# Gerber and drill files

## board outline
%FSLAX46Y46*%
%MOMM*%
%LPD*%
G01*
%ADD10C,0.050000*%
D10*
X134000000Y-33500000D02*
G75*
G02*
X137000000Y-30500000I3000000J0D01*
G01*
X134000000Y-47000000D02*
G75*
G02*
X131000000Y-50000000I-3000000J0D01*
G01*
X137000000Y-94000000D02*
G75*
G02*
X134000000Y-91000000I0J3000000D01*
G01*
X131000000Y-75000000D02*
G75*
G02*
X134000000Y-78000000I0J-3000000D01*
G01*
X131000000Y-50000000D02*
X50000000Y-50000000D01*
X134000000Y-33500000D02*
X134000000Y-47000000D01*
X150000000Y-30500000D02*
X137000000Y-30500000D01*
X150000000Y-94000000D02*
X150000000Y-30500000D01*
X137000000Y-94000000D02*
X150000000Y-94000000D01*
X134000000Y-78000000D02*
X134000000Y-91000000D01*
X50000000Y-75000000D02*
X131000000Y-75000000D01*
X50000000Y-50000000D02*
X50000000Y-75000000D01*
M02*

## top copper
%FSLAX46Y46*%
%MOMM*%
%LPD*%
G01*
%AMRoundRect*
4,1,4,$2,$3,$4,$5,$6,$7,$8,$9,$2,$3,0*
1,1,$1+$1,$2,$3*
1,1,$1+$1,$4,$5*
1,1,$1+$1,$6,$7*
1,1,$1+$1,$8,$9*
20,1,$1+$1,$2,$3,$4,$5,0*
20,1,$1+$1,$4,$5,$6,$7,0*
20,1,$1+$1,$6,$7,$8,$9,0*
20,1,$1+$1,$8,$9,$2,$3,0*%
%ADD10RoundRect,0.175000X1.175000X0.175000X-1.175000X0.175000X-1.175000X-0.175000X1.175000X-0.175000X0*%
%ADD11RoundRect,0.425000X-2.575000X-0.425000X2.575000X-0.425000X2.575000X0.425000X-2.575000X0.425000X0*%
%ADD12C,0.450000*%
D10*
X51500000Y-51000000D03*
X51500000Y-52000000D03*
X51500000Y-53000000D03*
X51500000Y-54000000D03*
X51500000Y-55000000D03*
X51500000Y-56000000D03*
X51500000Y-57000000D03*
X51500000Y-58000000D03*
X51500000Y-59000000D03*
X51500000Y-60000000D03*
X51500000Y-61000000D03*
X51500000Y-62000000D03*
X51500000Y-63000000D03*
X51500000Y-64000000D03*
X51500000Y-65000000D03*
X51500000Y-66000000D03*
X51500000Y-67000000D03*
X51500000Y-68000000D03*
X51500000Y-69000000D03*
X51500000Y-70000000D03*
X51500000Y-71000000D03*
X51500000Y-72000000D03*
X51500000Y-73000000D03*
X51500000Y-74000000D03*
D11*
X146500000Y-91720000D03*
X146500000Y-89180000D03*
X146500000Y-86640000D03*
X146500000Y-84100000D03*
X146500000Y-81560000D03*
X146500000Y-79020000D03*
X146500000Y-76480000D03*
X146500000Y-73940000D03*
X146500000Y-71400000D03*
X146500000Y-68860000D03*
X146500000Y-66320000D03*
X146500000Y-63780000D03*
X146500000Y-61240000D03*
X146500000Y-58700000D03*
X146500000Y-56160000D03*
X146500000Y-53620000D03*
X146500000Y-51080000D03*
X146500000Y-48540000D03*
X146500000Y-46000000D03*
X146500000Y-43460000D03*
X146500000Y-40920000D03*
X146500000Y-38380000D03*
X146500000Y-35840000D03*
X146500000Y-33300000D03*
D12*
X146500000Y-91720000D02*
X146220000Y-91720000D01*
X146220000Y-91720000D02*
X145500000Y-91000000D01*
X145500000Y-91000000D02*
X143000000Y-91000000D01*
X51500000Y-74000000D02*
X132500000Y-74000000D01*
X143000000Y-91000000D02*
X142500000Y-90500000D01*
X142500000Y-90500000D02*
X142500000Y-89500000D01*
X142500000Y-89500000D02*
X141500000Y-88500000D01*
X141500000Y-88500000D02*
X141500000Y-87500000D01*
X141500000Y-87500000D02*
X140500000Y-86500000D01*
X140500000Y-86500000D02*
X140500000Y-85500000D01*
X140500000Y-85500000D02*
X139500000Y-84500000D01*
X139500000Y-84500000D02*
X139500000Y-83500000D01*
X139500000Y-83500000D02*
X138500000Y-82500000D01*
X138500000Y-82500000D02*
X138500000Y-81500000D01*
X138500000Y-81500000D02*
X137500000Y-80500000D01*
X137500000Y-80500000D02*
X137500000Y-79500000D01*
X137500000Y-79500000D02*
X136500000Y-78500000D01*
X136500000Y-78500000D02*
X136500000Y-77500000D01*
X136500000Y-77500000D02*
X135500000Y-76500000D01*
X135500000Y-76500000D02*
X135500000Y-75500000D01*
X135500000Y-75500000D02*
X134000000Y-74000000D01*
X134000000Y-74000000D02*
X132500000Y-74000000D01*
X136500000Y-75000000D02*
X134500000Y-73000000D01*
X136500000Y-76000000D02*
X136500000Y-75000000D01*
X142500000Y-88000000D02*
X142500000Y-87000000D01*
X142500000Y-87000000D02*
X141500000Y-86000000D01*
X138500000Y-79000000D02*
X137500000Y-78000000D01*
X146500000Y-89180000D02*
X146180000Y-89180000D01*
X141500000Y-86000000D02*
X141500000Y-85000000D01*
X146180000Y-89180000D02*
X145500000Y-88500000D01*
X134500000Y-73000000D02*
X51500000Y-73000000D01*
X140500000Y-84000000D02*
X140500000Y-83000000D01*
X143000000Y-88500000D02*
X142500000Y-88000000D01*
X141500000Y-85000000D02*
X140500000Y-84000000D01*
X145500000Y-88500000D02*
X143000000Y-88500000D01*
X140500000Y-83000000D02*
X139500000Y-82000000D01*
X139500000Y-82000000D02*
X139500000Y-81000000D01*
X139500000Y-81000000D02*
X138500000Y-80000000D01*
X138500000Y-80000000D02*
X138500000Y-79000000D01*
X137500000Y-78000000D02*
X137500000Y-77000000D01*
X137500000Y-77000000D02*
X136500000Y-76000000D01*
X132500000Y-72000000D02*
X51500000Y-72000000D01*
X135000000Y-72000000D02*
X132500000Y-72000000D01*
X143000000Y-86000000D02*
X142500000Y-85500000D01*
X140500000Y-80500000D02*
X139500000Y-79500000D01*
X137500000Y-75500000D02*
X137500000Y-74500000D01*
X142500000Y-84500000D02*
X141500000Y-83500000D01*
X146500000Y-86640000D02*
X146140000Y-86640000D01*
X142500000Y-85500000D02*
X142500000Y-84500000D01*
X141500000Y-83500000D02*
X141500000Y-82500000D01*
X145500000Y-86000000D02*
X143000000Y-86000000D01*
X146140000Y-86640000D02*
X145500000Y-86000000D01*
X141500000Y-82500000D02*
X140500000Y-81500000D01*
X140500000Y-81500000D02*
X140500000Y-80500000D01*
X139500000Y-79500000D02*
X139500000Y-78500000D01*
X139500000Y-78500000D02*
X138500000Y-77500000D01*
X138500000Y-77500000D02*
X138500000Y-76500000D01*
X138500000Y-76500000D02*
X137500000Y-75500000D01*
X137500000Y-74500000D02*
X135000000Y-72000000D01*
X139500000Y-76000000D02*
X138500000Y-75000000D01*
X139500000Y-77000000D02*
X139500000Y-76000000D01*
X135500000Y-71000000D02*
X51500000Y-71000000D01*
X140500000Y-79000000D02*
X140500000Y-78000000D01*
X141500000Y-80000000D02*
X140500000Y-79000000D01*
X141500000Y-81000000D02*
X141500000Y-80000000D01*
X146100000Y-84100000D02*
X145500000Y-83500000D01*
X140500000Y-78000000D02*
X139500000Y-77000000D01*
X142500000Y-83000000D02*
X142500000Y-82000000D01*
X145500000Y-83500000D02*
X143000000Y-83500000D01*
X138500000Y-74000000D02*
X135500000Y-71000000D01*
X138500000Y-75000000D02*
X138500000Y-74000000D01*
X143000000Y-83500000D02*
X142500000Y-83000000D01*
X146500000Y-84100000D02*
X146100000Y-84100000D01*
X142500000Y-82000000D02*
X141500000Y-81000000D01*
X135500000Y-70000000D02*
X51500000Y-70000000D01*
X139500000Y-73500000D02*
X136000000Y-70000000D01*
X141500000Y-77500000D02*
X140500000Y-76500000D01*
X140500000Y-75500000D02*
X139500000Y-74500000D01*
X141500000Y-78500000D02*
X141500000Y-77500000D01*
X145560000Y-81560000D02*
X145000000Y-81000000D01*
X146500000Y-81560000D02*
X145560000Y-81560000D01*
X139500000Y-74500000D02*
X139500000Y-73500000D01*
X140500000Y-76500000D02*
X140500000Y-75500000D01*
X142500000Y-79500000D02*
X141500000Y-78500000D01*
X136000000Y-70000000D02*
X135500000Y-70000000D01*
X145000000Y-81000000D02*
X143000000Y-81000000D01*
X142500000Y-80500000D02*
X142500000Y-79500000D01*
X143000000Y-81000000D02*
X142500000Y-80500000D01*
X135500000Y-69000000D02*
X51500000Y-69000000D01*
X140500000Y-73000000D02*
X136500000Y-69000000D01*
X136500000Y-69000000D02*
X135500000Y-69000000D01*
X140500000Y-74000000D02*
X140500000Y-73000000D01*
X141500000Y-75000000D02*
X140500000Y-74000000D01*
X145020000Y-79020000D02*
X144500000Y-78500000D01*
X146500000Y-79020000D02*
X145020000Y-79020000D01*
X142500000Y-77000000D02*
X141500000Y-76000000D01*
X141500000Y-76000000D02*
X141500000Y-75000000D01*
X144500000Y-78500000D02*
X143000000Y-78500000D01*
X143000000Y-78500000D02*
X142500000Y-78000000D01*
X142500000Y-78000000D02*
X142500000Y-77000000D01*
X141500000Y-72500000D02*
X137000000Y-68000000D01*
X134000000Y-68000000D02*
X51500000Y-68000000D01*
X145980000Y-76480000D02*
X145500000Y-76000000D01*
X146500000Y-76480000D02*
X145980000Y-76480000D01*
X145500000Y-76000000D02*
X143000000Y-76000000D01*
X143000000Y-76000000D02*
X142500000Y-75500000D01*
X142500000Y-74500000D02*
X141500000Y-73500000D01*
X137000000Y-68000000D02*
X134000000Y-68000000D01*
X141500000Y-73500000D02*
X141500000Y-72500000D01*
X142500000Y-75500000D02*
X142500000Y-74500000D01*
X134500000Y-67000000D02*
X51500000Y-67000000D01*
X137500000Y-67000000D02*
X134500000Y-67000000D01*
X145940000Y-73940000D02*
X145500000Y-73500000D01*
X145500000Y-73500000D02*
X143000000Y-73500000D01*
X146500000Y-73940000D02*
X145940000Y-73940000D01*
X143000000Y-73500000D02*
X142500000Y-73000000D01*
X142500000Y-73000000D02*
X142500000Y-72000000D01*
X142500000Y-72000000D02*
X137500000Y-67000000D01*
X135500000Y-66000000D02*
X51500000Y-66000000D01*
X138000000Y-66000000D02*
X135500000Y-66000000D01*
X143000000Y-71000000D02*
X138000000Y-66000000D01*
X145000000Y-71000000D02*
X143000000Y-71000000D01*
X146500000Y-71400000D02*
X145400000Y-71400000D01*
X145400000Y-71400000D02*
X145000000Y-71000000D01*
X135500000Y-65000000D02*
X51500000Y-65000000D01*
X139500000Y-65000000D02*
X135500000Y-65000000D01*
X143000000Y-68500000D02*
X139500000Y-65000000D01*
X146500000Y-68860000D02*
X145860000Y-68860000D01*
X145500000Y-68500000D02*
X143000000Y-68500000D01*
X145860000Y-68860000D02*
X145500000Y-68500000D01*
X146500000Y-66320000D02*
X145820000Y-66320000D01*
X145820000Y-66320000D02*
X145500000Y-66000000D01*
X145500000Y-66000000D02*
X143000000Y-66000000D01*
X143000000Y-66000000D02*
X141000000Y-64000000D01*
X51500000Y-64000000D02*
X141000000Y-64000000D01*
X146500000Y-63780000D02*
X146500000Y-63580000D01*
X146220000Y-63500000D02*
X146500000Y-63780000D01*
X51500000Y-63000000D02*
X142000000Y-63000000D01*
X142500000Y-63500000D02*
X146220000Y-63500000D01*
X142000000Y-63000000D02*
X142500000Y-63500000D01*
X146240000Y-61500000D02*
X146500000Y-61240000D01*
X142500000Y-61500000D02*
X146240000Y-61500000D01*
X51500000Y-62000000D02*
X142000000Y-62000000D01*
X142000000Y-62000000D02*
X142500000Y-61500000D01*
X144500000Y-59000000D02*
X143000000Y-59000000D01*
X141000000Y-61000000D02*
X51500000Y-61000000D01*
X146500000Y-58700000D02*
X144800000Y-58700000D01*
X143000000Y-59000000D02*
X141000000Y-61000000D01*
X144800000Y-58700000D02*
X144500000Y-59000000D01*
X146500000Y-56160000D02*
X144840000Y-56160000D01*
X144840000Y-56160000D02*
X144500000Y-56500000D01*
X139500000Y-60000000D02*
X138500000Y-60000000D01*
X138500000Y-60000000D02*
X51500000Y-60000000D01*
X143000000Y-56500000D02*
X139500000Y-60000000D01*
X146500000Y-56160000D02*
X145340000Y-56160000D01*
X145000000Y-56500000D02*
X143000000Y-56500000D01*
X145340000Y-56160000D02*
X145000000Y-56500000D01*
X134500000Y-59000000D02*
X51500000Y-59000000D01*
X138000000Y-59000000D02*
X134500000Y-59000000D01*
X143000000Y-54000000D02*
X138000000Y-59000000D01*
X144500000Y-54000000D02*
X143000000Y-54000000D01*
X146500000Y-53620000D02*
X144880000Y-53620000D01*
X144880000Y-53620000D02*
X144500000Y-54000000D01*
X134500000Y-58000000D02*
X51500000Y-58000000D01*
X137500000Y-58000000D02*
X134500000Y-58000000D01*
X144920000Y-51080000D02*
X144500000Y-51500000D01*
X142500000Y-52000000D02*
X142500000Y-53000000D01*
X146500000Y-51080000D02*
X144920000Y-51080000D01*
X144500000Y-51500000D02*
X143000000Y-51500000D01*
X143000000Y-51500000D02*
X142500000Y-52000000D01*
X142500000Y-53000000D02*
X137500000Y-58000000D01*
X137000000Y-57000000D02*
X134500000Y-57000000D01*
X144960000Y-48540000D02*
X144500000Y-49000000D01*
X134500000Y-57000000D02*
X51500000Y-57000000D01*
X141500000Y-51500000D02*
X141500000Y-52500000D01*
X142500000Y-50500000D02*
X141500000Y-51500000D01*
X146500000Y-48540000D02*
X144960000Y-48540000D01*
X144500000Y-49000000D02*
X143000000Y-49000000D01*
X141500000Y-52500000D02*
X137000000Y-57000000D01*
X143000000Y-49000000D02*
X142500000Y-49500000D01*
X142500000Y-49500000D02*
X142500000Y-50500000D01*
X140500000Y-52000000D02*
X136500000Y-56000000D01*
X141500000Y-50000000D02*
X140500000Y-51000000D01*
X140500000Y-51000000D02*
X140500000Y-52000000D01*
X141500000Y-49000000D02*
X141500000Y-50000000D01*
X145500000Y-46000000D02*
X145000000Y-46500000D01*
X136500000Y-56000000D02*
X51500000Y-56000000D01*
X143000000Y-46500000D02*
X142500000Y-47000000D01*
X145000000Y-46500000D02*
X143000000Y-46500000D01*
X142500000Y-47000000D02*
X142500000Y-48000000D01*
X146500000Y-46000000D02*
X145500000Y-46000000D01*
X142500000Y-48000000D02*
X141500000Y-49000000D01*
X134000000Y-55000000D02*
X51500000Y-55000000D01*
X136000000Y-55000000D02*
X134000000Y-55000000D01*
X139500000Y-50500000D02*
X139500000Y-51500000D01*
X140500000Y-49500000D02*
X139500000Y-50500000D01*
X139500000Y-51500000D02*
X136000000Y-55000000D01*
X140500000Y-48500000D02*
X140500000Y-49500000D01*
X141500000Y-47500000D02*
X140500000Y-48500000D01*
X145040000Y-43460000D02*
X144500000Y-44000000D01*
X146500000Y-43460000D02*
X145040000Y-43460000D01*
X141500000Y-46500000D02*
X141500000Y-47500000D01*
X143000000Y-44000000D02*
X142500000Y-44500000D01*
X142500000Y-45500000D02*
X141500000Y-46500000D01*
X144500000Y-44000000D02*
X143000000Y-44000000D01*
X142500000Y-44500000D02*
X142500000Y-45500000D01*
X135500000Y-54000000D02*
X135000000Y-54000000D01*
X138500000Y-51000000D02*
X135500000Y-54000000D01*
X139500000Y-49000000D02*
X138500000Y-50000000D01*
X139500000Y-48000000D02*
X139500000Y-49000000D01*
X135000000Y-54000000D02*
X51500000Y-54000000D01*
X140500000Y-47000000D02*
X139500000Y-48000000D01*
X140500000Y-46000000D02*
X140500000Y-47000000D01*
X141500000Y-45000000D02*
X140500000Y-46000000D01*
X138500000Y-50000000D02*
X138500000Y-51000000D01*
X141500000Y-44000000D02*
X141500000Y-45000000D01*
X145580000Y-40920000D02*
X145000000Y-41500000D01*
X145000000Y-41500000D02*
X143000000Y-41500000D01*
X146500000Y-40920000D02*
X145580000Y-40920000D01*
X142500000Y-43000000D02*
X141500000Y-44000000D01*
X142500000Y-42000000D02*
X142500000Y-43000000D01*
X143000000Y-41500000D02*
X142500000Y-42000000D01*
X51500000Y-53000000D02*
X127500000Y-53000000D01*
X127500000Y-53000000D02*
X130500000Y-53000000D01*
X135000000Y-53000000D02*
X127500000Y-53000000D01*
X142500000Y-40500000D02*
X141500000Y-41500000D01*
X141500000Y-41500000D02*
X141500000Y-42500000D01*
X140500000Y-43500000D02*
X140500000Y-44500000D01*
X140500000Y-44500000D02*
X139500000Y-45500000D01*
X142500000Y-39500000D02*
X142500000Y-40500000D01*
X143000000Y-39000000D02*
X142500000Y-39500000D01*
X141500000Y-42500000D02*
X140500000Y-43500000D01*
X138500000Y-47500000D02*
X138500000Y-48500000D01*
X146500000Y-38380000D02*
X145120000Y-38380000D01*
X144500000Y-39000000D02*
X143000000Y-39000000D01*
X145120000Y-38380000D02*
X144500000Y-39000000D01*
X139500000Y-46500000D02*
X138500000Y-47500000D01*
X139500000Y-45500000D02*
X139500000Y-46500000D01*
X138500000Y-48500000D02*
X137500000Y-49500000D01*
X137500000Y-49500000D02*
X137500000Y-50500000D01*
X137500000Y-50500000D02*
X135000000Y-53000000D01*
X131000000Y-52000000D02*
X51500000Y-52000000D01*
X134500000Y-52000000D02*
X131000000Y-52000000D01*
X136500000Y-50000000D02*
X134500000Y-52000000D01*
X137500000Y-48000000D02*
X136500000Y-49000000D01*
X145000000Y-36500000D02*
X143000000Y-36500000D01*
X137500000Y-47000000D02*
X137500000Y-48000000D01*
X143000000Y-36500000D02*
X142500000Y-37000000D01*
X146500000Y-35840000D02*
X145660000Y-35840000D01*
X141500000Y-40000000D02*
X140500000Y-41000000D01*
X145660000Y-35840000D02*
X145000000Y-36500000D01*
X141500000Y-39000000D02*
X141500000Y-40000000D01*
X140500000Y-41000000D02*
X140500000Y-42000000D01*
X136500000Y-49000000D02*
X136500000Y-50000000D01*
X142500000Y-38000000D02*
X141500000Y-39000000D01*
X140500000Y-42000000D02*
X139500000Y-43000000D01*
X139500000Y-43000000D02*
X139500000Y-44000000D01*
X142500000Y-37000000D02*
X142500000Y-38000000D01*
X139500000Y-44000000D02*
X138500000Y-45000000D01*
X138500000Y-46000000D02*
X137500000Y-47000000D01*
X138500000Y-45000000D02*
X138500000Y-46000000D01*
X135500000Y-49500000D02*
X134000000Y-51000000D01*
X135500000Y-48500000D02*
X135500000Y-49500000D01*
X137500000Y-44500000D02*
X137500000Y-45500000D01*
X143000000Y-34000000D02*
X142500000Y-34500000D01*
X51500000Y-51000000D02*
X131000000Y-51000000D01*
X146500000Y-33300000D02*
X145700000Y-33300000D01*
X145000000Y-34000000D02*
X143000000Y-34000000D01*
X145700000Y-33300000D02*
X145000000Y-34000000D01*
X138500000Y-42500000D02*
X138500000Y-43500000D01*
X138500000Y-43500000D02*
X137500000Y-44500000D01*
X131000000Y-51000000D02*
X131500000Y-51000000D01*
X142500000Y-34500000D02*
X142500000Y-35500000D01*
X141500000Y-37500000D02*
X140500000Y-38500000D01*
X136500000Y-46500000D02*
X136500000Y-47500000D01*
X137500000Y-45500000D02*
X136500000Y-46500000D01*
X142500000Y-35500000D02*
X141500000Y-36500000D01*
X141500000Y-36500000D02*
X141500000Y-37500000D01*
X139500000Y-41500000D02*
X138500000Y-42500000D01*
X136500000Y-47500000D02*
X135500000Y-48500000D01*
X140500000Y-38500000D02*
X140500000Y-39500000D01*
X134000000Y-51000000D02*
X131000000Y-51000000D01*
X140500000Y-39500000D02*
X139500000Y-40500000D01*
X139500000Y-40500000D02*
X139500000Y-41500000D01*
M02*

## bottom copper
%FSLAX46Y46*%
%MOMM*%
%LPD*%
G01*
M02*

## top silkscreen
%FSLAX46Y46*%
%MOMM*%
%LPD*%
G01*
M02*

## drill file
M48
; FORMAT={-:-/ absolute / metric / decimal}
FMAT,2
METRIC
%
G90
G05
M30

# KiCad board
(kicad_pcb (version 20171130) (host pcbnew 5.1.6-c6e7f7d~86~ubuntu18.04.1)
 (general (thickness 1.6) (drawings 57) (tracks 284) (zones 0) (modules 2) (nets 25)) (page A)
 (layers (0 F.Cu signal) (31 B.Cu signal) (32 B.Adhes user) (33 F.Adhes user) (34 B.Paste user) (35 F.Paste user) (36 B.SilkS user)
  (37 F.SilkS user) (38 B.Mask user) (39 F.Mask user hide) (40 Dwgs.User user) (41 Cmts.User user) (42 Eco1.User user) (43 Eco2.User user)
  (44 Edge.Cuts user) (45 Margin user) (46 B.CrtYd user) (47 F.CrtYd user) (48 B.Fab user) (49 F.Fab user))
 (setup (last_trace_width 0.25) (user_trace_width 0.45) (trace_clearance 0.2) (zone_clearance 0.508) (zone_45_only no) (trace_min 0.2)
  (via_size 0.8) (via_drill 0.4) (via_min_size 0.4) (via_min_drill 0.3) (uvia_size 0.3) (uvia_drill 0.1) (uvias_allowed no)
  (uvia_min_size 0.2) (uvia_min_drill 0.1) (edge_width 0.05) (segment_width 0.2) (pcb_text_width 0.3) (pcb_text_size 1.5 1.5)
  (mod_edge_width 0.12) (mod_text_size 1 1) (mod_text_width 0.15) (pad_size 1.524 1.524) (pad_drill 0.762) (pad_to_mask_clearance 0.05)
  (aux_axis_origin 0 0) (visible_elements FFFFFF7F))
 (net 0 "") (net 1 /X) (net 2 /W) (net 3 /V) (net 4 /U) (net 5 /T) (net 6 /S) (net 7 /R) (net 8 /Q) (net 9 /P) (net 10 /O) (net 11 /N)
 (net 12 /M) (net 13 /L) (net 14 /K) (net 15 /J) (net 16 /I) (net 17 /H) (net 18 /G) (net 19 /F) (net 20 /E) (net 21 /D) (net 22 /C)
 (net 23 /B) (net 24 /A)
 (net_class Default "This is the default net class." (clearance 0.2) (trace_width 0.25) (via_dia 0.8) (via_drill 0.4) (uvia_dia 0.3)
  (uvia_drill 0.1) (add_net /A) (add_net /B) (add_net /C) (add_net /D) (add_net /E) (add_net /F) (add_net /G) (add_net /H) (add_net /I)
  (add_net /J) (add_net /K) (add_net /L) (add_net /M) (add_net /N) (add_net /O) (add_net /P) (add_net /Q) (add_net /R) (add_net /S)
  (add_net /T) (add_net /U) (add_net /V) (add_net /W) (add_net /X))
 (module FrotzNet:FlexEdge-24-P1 (layer F.Cu) (at 51.5 74 180)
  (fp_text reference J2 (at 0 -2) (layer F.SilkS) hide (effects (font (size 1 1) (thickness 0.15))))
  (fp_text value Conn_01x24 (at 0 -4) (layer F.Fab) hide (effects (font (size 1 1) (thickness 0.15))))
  (pad 24 smd roundrect (at 0 23 180) (size 2.7 0.7) (layers F.Cu F.Paste F.Mask) (roundrect_rratio 0.25) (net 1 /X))
  (pad 23 smd roundrect (at 0 22 180) (size 2.7 0.7) (layers F.Cu F.Paste F.Mask) (roundrect_rratio 0.25) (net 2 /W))
  (pad 22 smd roundrect (at 0 21 180) (size 2.7 0.7) (layers F.Cu F.Paste F.Mask) (roundrect_rratio 0.25) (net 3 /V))
  (pad 21 smd roundrect (at 0 20 180) (size 2.7 0.7) (layers F.Cu F.Paste F.Mask) (roundrect_rratio 0.25) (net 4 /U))
  (pad 20 smd roundrect (at 0 19 180) (size 2.7 0.7) (layers F.Cu F.Paste F.Mask) (roundrect_rratio 0.25) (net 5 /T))
  (pad 19 smd roundrect (at 0 18 180) (size 2.7 0.7) (layers F.Cu F.Paste F.Mask) (roundrect_rratio 0.25) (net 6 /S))
  (pad 18 smd roundrect (at 0 17 180) (size 2.7 0.7) (layers F.Cu F.Paste F.Mask) (roundrect_rratio 0.25) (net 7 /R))
  (pad 17 smd roundrect (at 0 16 180) (size 2.7 0.7) (layers F.Cu F.Paste F.Mask) (roundrect_rratio 0.25) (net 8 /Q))
  (pad 16 smd roundrect (at 0 15 180) (size 2.7 0.7) (layers F.Cu F.Paste F.Mask) (roundrect_rratio 0.25) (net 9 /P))
  (pad 15 smd roundrect (at 0 14 180) (size 2.7 0.7) (layers F.Cu F.Paste F.Mask) (roundrect_rratio 0.25) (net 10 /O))
  (pad 14 smd roundrect (at 0 13 180) (size 2.7 0.7) (layers F.Cu F.Paste F.Mask) (roundrect_rratio 0.25) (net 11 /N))
  (pad 13 smd roundrect (at 0 12 180) (size 2.7 0.7) (layers F.Cu F.Paste F.Mask) (roundrect_rratio 0.25) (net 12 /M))
  (pad 12 smd roundrect (at 0 11 180) (size 2.7 0.7) (layers F.Cu F.Paste F.Mask) (roundrect_rratio 0.25) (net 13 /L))
  (pad 11 smd roundrect (at 0 10 180) (size 2.7 0.7) (layers F.Cu F.Paste F.Mask) (roundrect_rratio 0.25) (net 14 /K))
  (pad 10 smd roundrect (at 0 9 180) (size 2.7 0.7) (layers F.Cu F.Paste F.Mask) (roundrect_rratio 0.25) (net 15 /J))
  (pad 9 smd roundrect (at 0 8 180) (size 2.7 0.7) (layers F.Cu F.Paste F.Mask) (roundrect_rratio 0.25) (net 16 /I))
  (pad 8 smd roundrect (at 0 7 180) (size 2.7 0.7) (layers F.Cu F.Paste F.Mask) (roundrect_rratio 0.25) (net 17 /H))
  (pad 7 smd roundrect (at 0 6 180) (size 2.7 0.7) (layers F.Cu F.Paste F.Mask) (roundrect_rratio 0.25) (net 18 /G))
  (pad 6 smd roundrect (at 0 5 180) (size 2.7 0.7) (layers F.Cu F.Paste F.Mask) (roundrect_rratio 0.25) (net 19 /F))
  (pad 5 smd roundrect (at 0 4 180) (size 2.7 0.7) (layers F.Cu F.Paste F.Mask) (roundrect_rratio 0.25) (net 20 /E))
  (pad 4 smd roundrect (at 0 3 180) (size 2.7 0.7) (layers F.Cu F.Paste F.Mask) (roundrect_rratio 0.25) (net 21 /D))
  (pad 3 smd roundrect (at 0 2 180) (size 2.7 0.7) (layers F.Cu F.Paste F.Mask) (roundrect_rratio 0.25) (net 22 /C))
  (pad 2 smd roundrect (at 0 1 180) (size 2.7 0.7) (layers F.Cu F.Paste F.Mask) (roundrect_rratio 0.25) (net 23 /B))
  (pad 1 smd roundrect (at 0 0 180) (size 2.7 0.7) (layers F.Cu F.Paste F.Mask) (roundrect_rratio 0.25) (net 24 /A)))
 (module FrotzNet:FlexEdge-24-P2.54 (layer F.Cu) (at 146.5 33.3)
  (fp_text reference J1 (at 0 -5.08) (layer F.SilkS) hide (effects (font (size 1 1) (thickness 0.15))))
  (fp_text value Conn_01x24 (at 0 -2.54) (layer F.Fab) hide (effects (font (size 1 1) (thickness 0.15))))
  (pad 24 smd roundrect (at 0 58.42) (size 6 1.7) (layers F.Cu F.Paste F.Mask) (roundrect_rratio 0.25) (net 24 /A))
  (pad 23 smd roundrect (at 0 55.88) (size 6 1.7) (layers F.Cu F.Paste F.Mask) (roundrect_rratio 0.25) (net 23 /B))
  (pad 22 smd roundrect (at 0 53.34) (size 6 1.7) (layers F.Cu F.Paste F.Mask) (roundrect_rratio 0.25) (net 22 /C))
  (pad 21 smd roundrect (at 0 50.8) (size 6 1.7) (layers F.Cu F.Paste F.Mask) (roundrect_rratio 0.25) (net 21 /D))
  (pad 20 smd roundrect (at 0 48.26) (size 6 1.7) (layers F.Cu F.Paste F.Mask) (roundrect_rratio 0.25) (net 20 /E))
  (pad 19 smd roundrect (at 0 45.72) (size 6 1.7) (layers F.Cu F.Paste F.Mask) (roundrect_rratio 0.25) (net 19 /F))
  (pad 18 smd roundrect (at 0 43.18) (size 6 1.7) (layers F.Cu F.Paste F.Mask) (roundrect_rratio 0.25) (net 18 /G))
  (pad 17 smd roundrect (at 0 40.64) (size 6 1.7) (layers F.Cu F.Paste F.Mask) (roundrect_rratio 0.25) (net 17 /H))
  (pad 16 smd roundrect (at 0 38.1) (size 6 1.7) (layers F.Cu F.Paste F.Mask) (roundrect_rratio 0.25) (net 16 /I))
  (pad 15 smd roundrect (at 0 35.56) (size 6 1.7) (layers F.Cu F.Paste F.Mask) (roundrect_rratio 0.25) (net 15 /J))
  (pad 14 smd roundrect (at 0 33.02) (size 6 1.7) (layers F.Cu F.Paste F.Mask) (roundrect_rratio 0.25) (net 14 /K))
  (pad 13 smd roundrect (at 0 30.48) (size 6 1.7) (layers F.Cu F.Paste F.Mask) (roundrect_rratio 0.25) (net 13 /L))
  (pad 12 smd roundrect (at 0 27.94) (size 6 1.7) (layers F.Cu F.Paste F.Mask) (roundrect_rratio 0.25) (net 12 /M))
  (pad 11 smd roundrect (at 0 25.4) (size 6 1.7) (layers F.Cu F.Paste F.Mask) (roundrect_rratio 0.25) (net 11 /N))
  (pad 10 smd roundrect (at 0 22.86) (size 6 1.7) (layers F.Cu F.Paste F.Mask) (roundrect_rratio 0.25) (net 10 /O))
  (pad 9 smd roundrect (at 0 20.32) (size 6 1.7) (layers F.Cu F.Paste F.Mask) (roundrect_rratio 0.25) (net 9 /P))
  (pad 8 smd roundrect (at 0 17.78) (size 6 1.7) (layers F.Cu F.Paste F.Mask) (roundrect_rratio 0.25) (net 8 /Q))
  (pad 7 smd roundrect (at 0 15.24) (size 6 1.7) (layers F.Cu F.Paste F.Mask) (roundrect_rratio 0.25) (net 7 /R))
  (pad 6 smd roundrect (at 0 12.7) (size 6 1.7) (layers F.Cu F.Paste F.Mask) (roundrect_rratio 0.25) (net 6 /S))
  (pad 5 smd roundrect (at 0 10.16) (size 6 1.7) (layers F.Cu F.Paste F.Mask) (roundrect_rratio 0.25) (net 5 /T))
  (pad 4 smd roundrect (at 0 7.62) (size 6 1.7) (layers F.Cu F.Paste F.Mask) (roundrect_rratio 0.25) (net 4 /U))
  (pad 3 smd roundrect (at 0 5.08) (size 6 1.7) (layers F.Cu F.Paste F.Mask) (roundrect_rratio 0.25) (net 3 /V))
  (pad 2 smd roundrect (at 0 2.54) (size 6 1.7) (layers F.Cu F.Paste F.Mask) (roundrect_rratio 0.25) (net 2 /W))
  (pad 1 smd roundrect (at 0 0) (size 6 1.7) (layers F.Cu F.Paste F.Mask) (roundrect_rratio 0.25) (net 1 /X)))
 (gr_arc (start 137 33.5) (end 137 30.5) (angle -90) (layer Edge.Cuts) (width 0.05))
 (gr_arc (start 131 47) (end 131 50) (angle -90) (layer Edge.Cuts) (width 0.05))
 (gr_arc (start 137 91) (end 134 91) (angle -90) (layer Edge.Cuts) (width 0.05))
 (gr_arc (start 131 78) (end 134 78) (angle -90) (layer Edge.Cuts) (width 0.05))
 (gr_line (start 131 50) (end 50 50) (layer Edge.Cuts) (width 0.05))
 (gr_line (start 134 33.5) (end 134 47) (layer Edge.Cuts) (width 0.05))
 (gr_line (start 150 30.5) (end 137 30.5) (layer Edge.Cuts) (width 0.05))
 (gr_line (start 150 94) (end 150 30.5) (layer Edge.Cuts) (width 0.05))
 (gr_line (start 137 94) (end 150 94) (layer Edge.Cuts) (width 0.05))
 (gr_line (start 134 78) (end 134 91) (layer Edge.Cuts) (width 0.05))
 (gr_line (start 50 75) (end 131 75) (layer Edge.Cuts) (width 0.05))
 (gr_line (start 50 50) (end 50 75) (layer Edge.Cuts) (width 0.05))
 (segment (start 146.5 91.72) (end 146.22 91.72) (width 0.45) (layer F.Cu) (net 24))
 (segment (start 146.22 91.72) (end 145.5 91) (width 0.45) (layer F.Cu) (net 24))
 (segment (start 145.5 91) (end 143 91) (width 0.45) (layer F.Cu) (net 24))
 (segment (start 51.5 74) (end 132.5 74) (width 0.45) (layer F.Cu) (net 24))
 (segment (start 143 91) (end 142.5 90.5) (width 0.45) (layer F.Cu) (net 24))
 (segment (start 142.5 90.5) (end 142.5 89.5) (width 0.45) (layer F.Cu) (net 24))
 (segment (start 142.5 89.5) (end 141.5 88.5) (width 0.45) (layer F.Cu) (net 24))
 (segment (start 141.5 88.5) (end 141.5 87.5) (width 0.45) (layer F.Cu) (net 24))
 (segment (start 141.5 87.5) (end 140.5 86.5) (width 0.45) (layer F.Cu) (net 24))
 (segment (start 140.5 86.5) (end 140.5 85.5) (width 0.45) (layer F.Cu) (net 24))
 (segment (start 140.5 85.5) (end 139.5 84.5) (width 0.45) (layer F.Cu) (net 24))
 (segment (start 139.5 84.5) (end 139.5 83.5) (width 0.45) (layer F.Cu) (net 24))
 (segment (start 139.5 83.5) (end 138.5 82.5) (width 0.45) (layer F.Cu) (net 24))
 (segment (start 138.5 82.5) (end 138.5 81.5) (width 0.45) (layer F.Cu) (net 24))
 (segment (start 138.5 81.5) (end 137.5 80.5) (width 0.45) (layer F.Cu) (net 24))
 (segment (start 137.5 80.5) (end 137.5 79.5) (width 0.45) (layer F.Cu) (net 24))
 (segment (start 137.5 79.5) (end 136.5 78.5) (width 0.45) (layer F.Cu) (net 24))
 (segment (start 136.5 78.5) (end 136.5 77.5) (width 0.45) (layer F.Cu) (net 24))
 (segment (start 136.5 77.5) (end 135.5 76.5) (width 0.45) (layer F.Cu) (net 24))
 (segment (start 135.5 76.5) (end 135.5 75.5) (width 0.45) (layer F.Cu) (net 24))
 (segment (start 135.5 75.5) (end 134 74) (width 0.45) (layer F.Cu) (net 24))
 (segment (start 134 74) (end 132.5 74) (width 0.45) (layer F.Cu) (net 24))
 (segment (start 136.5 75) (end 134.5 73) (width 0.45) (layer F.Cu) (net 23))
 (segment (start 136.5 76) (end 136.5 75) (width 0.45) (layer F.Cu) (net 23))
 (segment (start 142.5 88) (end 142.5 87) (width 0.45) (layer F.Cu) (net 23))
 (segment (start 142.5 87) (end 141.5 86) (width 0.45) (layer F.Cu) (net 23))
 (segment (start 138.5 79) (end 137.5 78) (width 0.45) (layer F.Cu) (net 23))
 (segment (start 146.5 89.18) (end 146.18 89.18) (width 0.45) (layer F.Cu) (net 23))
 (segment (start 141.5 86) (end 141.5 85) (width 0.45) (layer F.Cu) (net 23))
 (segment (start 146.18 89.18) (end 145.5 88.5) (width 0.45) (layer F.Cu) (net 23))
 (segment (start 134.5 73) (end 51.5 73) (width 0.45) (layer F.Cu) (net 23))
 (segment (start 140.5 84) (end 140.5 83) (width 0.45) (layer F.Cu) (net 23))
 (segment (start 143 88.5) (end 142.5 88) (width 0.45) (layer F.Cu) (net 23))
 (segment (start 141.5 85) (end 140.5 84) (width 0.45) (layer F.Cu) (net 23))
 (segment (start 145.5 88.5) (end 143 88.5) (width 0.45) (layer F.Cu) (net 23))
 (segment (start 140.5 83) (end 139.5 82) (width 0.45) (layer F.Cu) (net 23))
 (segment (start 139.5 82) (end 139.5 81) (width 0.45) (layer F.Cu) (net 23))
 (segment (start 139.5 81) (end 138.5 80) (width 0.45) (layer F.Cu) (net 23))
 (segment (start 138.5 80) (end 138.5 79) (width 0.45) (layer F.Cu) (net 23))
 (segment (start 137.5 78) (end 137.5 77) (width 0.45) (layer F.Cu) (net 23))
 (segment (start 137.5 77) (end 136.5 76) (width 0.45) (layer F.Cu) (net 23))
 (segment (start 132.5 72) (end 51.5 72) (width 0.45) (layer F.Cu) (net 22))
 (segment (start 135 72) (end 132.5 72) (width 0.45) (layer F.Cu) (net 22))
 (segment (start 143 86) (end 142.5 85.5) (width 0.45) (layer F.Cu) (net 22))
 (segment (start 140.5 80.5) (end 139.5 79.5) (width 0.45) (layer F.Cu) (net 22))
 (segment (start 137.5 75.5) (end 137.5 74.5) (width 0.45) (layer F.Cu) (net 22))
 (segment (start 142.5 84.5) (end 141.5 83.5) (width 0.45) (layer F.Cu) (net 22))
 (segment (start 146.5 86.64) (end 146.14 86.64) (width 0.45) (layer F.Cu) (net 22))
 (segment (start 142.5 85.5) (end 142.5 84.5) (width 0.45) (layer F.Cu) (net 22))
 (segment (start 141.5 83.5) (end 141.5 82.5) (width 0.45) (layer F.Cu) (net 22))
 (segment (start 145.5 86) (end 143 86) (width 0.45) (layer F.Cu) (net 22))
 (segment (start 146.14 86.64) (end 145.5 86) (width 0.45) (layer F.Cu) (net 22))
 (segment (start 141.5 82.5) (end 140.5 81.5) (width 0.45) (layer F.Cu) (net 22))
 (segment (start 140.5 81.5) (end 140.5 80.5) (width 0.45) (layer F.Cu) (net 22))
 (segment (start 139.5 79.5) (end 139.5 78.5) (width 0.45) (layer F.Cu) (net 22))
 (segment (start 139.5 78.5) (end 138.5 77.5) (width 0.45) (layer F.Cu) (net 22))
 (segment (start 138.5 77.5) (end 138.5 76.5) (width 0.45) (layer F.Cu) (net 22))
 (segment (start 138.5 76.5) (end 137.5 75.5) (width 0.45) (layer F.Cu) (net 22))
 (segment (start 137.5 74.5) (end 135 72) (width 0.45) (layer F.Cu) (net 22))
 (segment (start 139.5 76) (end 138.5 75) (width 0.45) (layer F.Cu) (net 21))
 (segment (start 139.5 77) (end 139.5 76) (width 0.45) (layer F.Cu) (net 21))
 (segment (start 135.5 71) (end 51.5 71) (width 0.45) (layer F.Cu) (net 21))
 (segment (start 140.5 79) (end 140.5 78) (width 0.45) (layer F.Cu) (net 21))
 (segment (start 141.5 80) (end 140.5 79) (width 0.45) (layer F.Cu) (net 21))
 (segment (start 141.5 81) (end 141.5 80) (width 0.45) (layer F.Cu) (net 21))
 (segment (start 146.1 84.1) (end 145.5 83.5) (width 0.45) (layer F.Cu) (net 21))
 (segment (start 140.5 78) (end 139.5 77) (width 0.45) (layer F.Cu) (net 21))
 (segment (start 142.5 83) (end 142.5 82) (width 0.45) (layer F.Cu) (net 21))
 (segment (start 145.5 83.5) (end 143 83.5) (width 0.45) (layer F.Cu) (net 21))
 (segment (start 138.5 74) (end 135.5 71) (width 0.45) (layer F.Cu) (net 21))
 (segment (start 138.5 75) (end 138.5 74) (width 0.45) (layer F.Cu) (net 21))
 (segment (start 143 83.5) (end 142.5 83) (width 0.45) (layer F.Cu) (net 21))
 (segment (start 146.5 84.1) (end 146.1 84.1) (width 0.45) (layer F.Cu) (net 21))
 (segment (start 142.5 82) (end 141.5 81) (width 0.45) (layer F.Cu) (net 21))
 (segment (start 135.5 70) (end 51.5 70) (width 0.45) (layer F.Cu) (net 20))
 (segment (start 139.5 73.5) (end 136 70) (width 0.45) (layer F.Cu) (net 20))
 (segment (start 141.5 77.5) (end 140.5 76.5) (width 0.45) (layer F.Cu) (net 20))
 (segment (start 140.5 75.5) (end 139.5 74.5) (width 0.45) (layer F.Cu) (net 20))
 (segment (start 141.5 78.5) (end 141.5 77.5) (width 0.45) (layer F.Cu) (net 20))
 (segment (start 145.56 81.56) (end 145 81) (width 0.45) (layer F.Cu) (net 20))
 (segment (start 146.5 81.56) (end 145.56 81.56) (width 0.45) (layer F.Cu) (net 20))
 (segment (start 139.5 74.5) (end 139.5 73.5) (width 0.45) (layer F.Cu) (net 20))
 (segment (start 140.5 76.5) (end 140.5 75.5) (width 0.45) (layer F.Cu) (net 20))
 (segment (start 142.5 79.5) (end 141.5 78.5) (width 0.45) (layer F.Cu) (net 20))
 (segment (start 136 70) (end 135.5 70) (width 0.45) (layer F.Cu) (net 20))
 (segment (start 145 81) (end 143 81) (width 0.45) (layer F.Cu) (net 20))
 (segment (start 142.5 80.5) (end 142.5 79.5) (width 0.45) (layer F.Cu) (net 20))
 (segment (start 143 81) (end 142.5 80.5) (width 0.45) (layer F.Cu) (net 20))
 (segment (start 135.5 69) (end 51.5 69) (width 0.45) (layer F.Cu) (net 19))
 (segment (start 140.5 73) (end 136.5 69) (width 0.45) (layer F.Cu) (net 19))
 (segment (start 136.5 69) (end 135.5 69) (width 0.45) (layer F.Cu) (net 19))
 (segment (start 140.5 74) (end 140.5 73) (width 0.45) (layer F.Cu) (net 19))
 (segment (start 141.5 75) (end 140.5 74) (width 0.45) (layer F.Cu) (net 19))
 (segment (start 145.02 79.02) (end 144.5 78.5) (width 0.45) (layer F.Cu) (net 19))
 (segment (start 146.5 79.02) (end 145.02 79.02) (width 0.45) (layer F.Cu) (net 19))
 (segment (start 142.5 77) (end 141.5 76) (width 0.45) (layer F.Cu) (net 19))
 (segment (start 141.5 76) (end 141.5 75) (width 0.45) (layer F.Cu) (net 19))
 (segment (start 144.5 78.5) (end 143 78.5) (width 0.45) (layer F.Cu) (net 19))
 (segment (start 143 78.5) (end 142.5 78) (width 0.45) (layer F.Cu) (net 19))
 (segment (start 142.5 78) (end 142.5 77) (width 0.45) (layer F.Cu) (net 19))
 (segment (start 141.5 72.5) (end 137 68) (width 0.45) (layer F.Cu) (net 18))
 (segment (start 134 68) (end 51.5 68) (width 0.45) (layer F.Cu) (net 18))
 (segment (start 145.98 76.48) (end 145.5 76) (width 0.45) (layer F.Cu) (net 18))
 (segment (start 146.5 76.48) (end 145.98 76.48) (width 0.45) (layer F.Cu) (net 18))
 (segment (start 145.5 76) (end 143 76) (width 0.45) (layer F.Cu) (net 18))
 (segment (start 143 76) (end 142.5 75.5) (width 0.45) (layer F.Cu) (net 18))
 (segment (start 142.5 74.5) (end 141.5 73.5) (width 0.45) (layer F.Cu) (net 18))
 (segment (start 137 68) (end 134 68) (width 0.45) (layer F.Cu) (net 18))
 (segment (start 141.5 73.5) (end 141.5 72.5) (width 0.45) (layer F.Cu) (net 18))
 (segment (start 142.5 75.5) (end 142.5 74.5) (width 0.45) (layer F.Cu) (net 18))
 (segment (start 134.5 67) (end 51.5 67) (width 0.45) (layer F.Cu) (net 17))
 (segment (start 137.5 67) (end 134.5 67) (width 0.45) (layer F.Cu) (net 17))
 (segment (start 145.94 73.94) (end 145.5 73.5) (width 0.45) (layer F.Cu) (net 17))
 (segment (start 145.5 73.5) (end 143 73.5) (width 0.45) (layer F.Cu) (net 17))
 (segment (start 146.5 73.94) (end 145.94 73.94) (width 0.45) (layer F.Cu) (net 17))
 (segment (start 143 73.5) (end 142.5 73) (width 0.45) (layer F.Cu) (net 17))
 (segment (start 142.5 73) (end 142.5 72) (width 0.45) (layer F.Cu) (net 17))
 (segment (start 142.5 72) (end 137.5 67) (width 0.45) (layer F.Cu) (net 17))
 (segment (start 135.5 66) (end 51.5 66) (width 0.45) (layer F.Cu) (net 16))
 (segment (start 138 66) (end 135.5 66) (width 0.45) (layer F.Cu) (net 16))
 (segment (start 143 71) (end 138 66) (width 0.45) (layer F.Cu) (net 16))
 (segment (start 145 71) (end 143 71) (width 0.45) (layer F.Cu) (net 16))
 (segment (start 146.5 71.4) (end 145.4 71.4) (width 0.45) (layer F.Cu) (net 16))
 (segment (start 145.4 71.4) (end 145 71) (width 0.45) (layer F.Cu) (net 16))
 (segment (start 135.5 65) (end 51.5 65) (width 0.45) (layer F.Cu) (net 15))
 (segment (start 139.5 65) (end 135.5 65) (width 0.45) (layer F.Cu) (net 15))
 (segment (start 143 68.5) (end 139.5 65) (width 0.45) (layer F.Cu) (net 15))
 (segment (start 146.5 68.86) (end 145.86 68.86) (width 0.45) (layer F.Cu) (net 15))
 (segment (start 145.5 68.5) (end 143 68.5) (width 0.45) (layer F.Cu) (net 15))
 (segment (start 145.86 68.86) (end 145.5 68.5) (width 0.45) (layer F.Cu) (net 15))
 (segment (start 146.5 66.32) (end 145.82 66.32) (width 0.45) (layer F.Cu) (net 14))
 (segment (start 145.82 66.32) (end 145.5 66) (width 0.45) (layer F.Cu) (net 14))
 (segment (start 145.5 66) (end 143 66) (width 0.45) (layer F.Cu) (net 14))
 (segment (start 143 66) (end 141 64) (width 0.45) (layer F.Cu) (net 14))
 (segment (start 51.5 64) (end 141 64) (width 0.45) (layer F.Cu) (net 14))
 (segment (start 146.5 63.78) (end 146.5 63.58) (width 0.45) (layer F.Cu) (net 13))
 (segment (start 146.22 63.5) (end 146.5 63.78) (width 0.45) (layer F.Cu) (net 13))
 (segment (start 51.5 63) (end 142 63) (width 0.45) (layer F.Cu) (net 13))
 (segment (start 142.5 63.5) (end 146.22 63.5) (width 0.45) (layer F.Cu) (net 13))
 (segment (start 142 63) (end 142.5 63.5) (width 0.45) (layer F.Cu) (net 13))
 (segment (start 146.24 61.5) (end 146.5 61.24) (width 0.45) (layer F.Cu) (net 12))
 (segment (start 142.5 61.5) (end 146.24 61.5) (width 0.45) (layer F.Cu) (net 12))
 (segment (start 51.5 62) (end 142 62) (width 0.45) (layer F.Cu) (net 12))
 (segment (start 142 62) (end 142.5 61.5) (width 0.45) (layer F.Cu) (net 12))
 (segment (start 144.5 59) (end 143 59) (width 0.45) (layer F.Cu) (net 11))
 (segment (start 141 61) (end 51.5 61) (width 0.45) (layer F.Cu) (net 11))
 (segment (start 146.5 58.7) (end 144.8 58.7) (width 0.45) (layer F.Cu) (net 11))
 (segment (start 143 59) (end 141 61) (width 0.45) (layer F.Cu) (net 11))
 (segment (start 144.8 58.7) (end 144.5 59) (width 0.45) (layer F.Cu) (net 11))
 (segment (start 146.5 56.16) (end 144.84 56.16) (width 0.45) (layer F.Cu) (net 10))
 (segment (start 144.84 56.16) (end 144.5 56.5) (width 0.45) (layer F.Cu) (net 10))
 (segment (start 139.5 60) (end 138.5 60) (width 0.45) (layer F.Cu) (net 10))
 (segment (start 138.5 60) (end 51.5 60) (width 0.45) (layer F.Cu) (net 10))
 (segment (start 143 56.5) (end 139.5 60) (width 0.45) (layer F.Cu) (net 10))
 (segment (start 146.5 56.16) (end 145.34 56.16) (width 0.45) (layer F.Cu) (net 10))
 (segment (start 145 56.5) (end 143 56.5) (width 0.45) (layer F.Cu) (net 10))
 (segment (start 145.34 56.16) (end 145 56.5) (width 0.45) (layer F.Cu) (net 10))
 (segment (start 134.5 59) (end 51.5 59) (width 0.45) (layer F.Cu) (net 9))
 (segment (start 138 59) (end 134.5 59) (width 0.45) (layer F.Cu) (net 9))
 (segment (start 143 54) (end 138 59) (width 0.45) (layer F.Cu) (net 9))
 (segment (start 144.5 54) (end 143 54) (width 0.45) (layer F.Cu) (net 9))
 (segment (start 146.5 53.62) (end 144.88 53.62) (width 0.45) (layer F.Cu) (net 9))
 (segment (start 144.88 53.62) (end 144.5 54) (width 0.45) (layer F.Cu) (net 9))
 (segment (start 134.5 58) (end 51.5 58) (width 0.45) (layer F.Cu) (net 8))
 (segment (start 137.5 58) (end 134.5 58) (width 0.45) (layer F.Cu) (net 8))
 (segment (start 144.92 51.08) (end 144.5 51.5) (width 0.45) (layer F.Cu) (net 8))
 (segment (start 142.5 52) (end 142.5 53) (width 0.45) (layer F.Cu) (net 8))
 (segment (start 146.5 51.08) (end 144.92 51.08) (width 0.45) (layer F.Cu) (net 8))
 (segment (start 144.5 51.5) (end 143 51.5) (width 0.45) (layer F.Cu) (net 8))
 (segment (start 143 51.5) (end 142.5 52) (width 0.45) (layer F.Cu) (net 8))
 (segment (start 142.5 53) (end 137.5 58) (width 0.45) (layer F.Cu) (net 8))
 (segment (start 137 57) (end 134.5 57) (width 0.45) (layer F.Cu) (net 7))
 (segment (start 144.96 48.54) (end 144.5 49) (width 0.45) (layer F.Cu) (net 7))
 (segment (start 134.5 57) (end 51.5 57) (width 0.45) (layer F.Cu) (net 7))
 (segment (start 141.5 51.5) (end 141.5 52.5) (width 0.45) (layer F.Cu) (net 7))
 (segment (start 142.5 50.5) (end 141.5 51.5) (width 0.45) (layer F.Cu) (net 7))
 (segment (start 146.5 48.54) (end 144.96 48.54) (width 0.45) (layer F.Cu) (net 7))
 (segment (start 144.5 49) (end 143 49) (width 0.45) (layer F.Cu) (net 7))
 (segment (start 141.5 52.5) (end 137 57) (width 0.45) (layer F.Cu) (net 7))
 (segment (start 143 49) (end 142.5 49.5) (width 0.45) (layer F.Cu) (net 7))
 (segment (start 142.5 49.5) (end 142.5 50.5) (width 0.45) (layer F.Cu) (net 7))
 (segment (start 140.5 52) (end 136.5 56) (width 0.45) (layer F.Cu) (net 6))
 (segment (start 141.5 50) (end 140.5 51) (width 0.45) (layer F.Cu) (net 6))
 (segment (start 140.5 51) (end 140.5 52) (width 0.45) (layer F.Cu) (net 6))
 (segment (start 141.5 49) (end 141.5 50) (width 0.45) (layer F.Cu) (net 6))
 (segment (start 145.5 46) (end 145 46.5) (width 0.45) (layer F.Cu) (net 6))
 (segment (start 136.5 56) (end 51.5 56) (width 0.45) (layer F.Cu) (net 6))
 (segment (start 143 46.5) (end 142.5 47) (width 0.45) (layer F.Cu) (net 6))
 (segment (start 145 46.5) (end 143 46.5) (width 0.45) (layer F.Cu) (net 6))
 (segment (start 142.5 47) (end 142.5 48) (width 0.45) (layer F.Cu) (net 6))
 (segment (start 146.5 46) (end 145.5 46) (width 0.45) (layer F.Cu) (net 6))
 (segment (start 142.5 48) (end 141.5 49) (width 0.45) (layer F.Cu) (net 6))
 (segment (start 134 55) (end 51.5 55) (width 0.45) (layer F.Cu) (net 5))
 (segment (start 136 55) (end 134 55) (width 0.45) (layer F.Cu) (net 5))
 (segment (start 139.5 50.5) (end 139.5 51.5) (width 0.45) (layer F.Cu) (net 5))
 (segment (start 140.5 49.5) (end 139.5 50.5) (width 0.45) (layer F.Cu) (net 5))
 (segment (start 139.5 51.5) (end 136 55) (width 0.45) (layer F.Cu) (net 5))
 (segment (start 140.5 48.5) (end 140.5 49.5) (width 0.45) (layer F.Cu) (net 5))
 (segment (start 141.5 47.5) (end 140.5 48.5) (width 0.45) (layer F.Cu) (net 5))
 (segment (start 145.04 43.46) (end 144.5 44) (width 0.45) (layer F.Cu) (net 5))
 (segment (start 146.5 43.46) (end 145.04 43.46) (width 0.45) (layer F.Cu) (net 5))
 (segment (start 141.5 46.5) (end 141.5 47.5) (width 0.45) (layer F.Cu) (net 5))
 (segment (start 143 44) (end 142.5 44.5) (width 0.45) (layer F.Cu) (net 5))
 (segment (start 142.5 45.5) (end 141.5 46.5) (width 0.45) (layer F.Cu) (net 5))
 (segment (start 144.5 44) (end 143 44) (width 0.45) (layer F.Cu) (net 5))
 (segment (start 142.5 44.5) (end 142.5 45.5) (width 0.45) (layer F.Cu) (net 5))
 (segment (start 135.5 54) (end 135 54) (width 0.45) (layer F.Cu) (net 4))
 (segment (start 138.5 51) (end 135.5 54) (width 0.45) (layer F.Cu) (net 4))
 (segment (start 139.5 49) (end 138.5 50) (width 0.45) (layer F.Cu) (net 4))
 (segment (start 139.5 48) (end 139.5 49) (width 0.45) (layer F.Cu) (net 4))
 (segment (start 135 54) (end 51.5 54) (width 0.45) (layer F.Cu) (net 4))
 (segment (start 140.5 47) (end 139.5 48) (width 0.45) (layer F.Cu) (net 4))
 (segment (start 140.5 46) (end 140.5 47) (width 0.45) (layer F.Cu) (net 4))
 (segment (start 141.5 45) (end 140.5 46) (width 0.45) (layer F.Cu) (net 4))
 (segment (start 138.5 50) (end 138.5 51) (width 0.45) (layer F.Cu) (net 4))
 (segment (start 141.5 44) (end 141.5 45) (width 0.45) (layer F.Cu) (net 4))
 (segment (start 145.58 40.92) (end 145 41.5) (width 0.45) (layer F.Cu) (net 4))
 (segment (start 145 41.5) (end 143 41.5) (width 0.45) (layer F.Cu) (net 4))
 (segment (start 146.5 40.92) (end 145.58 40.92) (width 0.45) (layer F.Cu) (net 4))
 (segment (start 142.5 43) (end 141.5 44) (width 0.45) (layer F.Cu) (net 4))
 (segment (start 142.5 42) (end 142.5 43) (width 0.45) (layer F.Cu) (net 4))
 (segment (start 143 41.5) (end 142.5 42) (width 0.45) (layer F.Cu) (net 4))
 (segment (start 51.5 53) (end 127.5 53) (width 0.45) (layer F.Cu) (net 3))
 (segment (start 127.5 53) (end 130.5 53) (width 0.45) (layer F.Cu) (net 3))
 (segment (start 135 53) (end 127.5 53) (width 0.45) (layer F.Cu) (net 3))
 (segment (start 142.5 40.5) (end 141.5 41.5) (width 0.45) (layer F.Cu) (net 3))
 (segment (start 141.5 41.5) (end 141.5 42.5) (width 0.45) (layer F.Cu) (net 3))
 (segment (start 140.5 43.5) (end 140.5 44.5) (width 0.45) (layer F.Cu) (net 3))
 (segment (start 140.5 44.5) (end 139.5 45.5) (width 0.45) (layer F.Cu) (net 3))
 (segment (start 142.5 39.5) (end 142.5 40.5) (width 0.45) (layer F.Cu) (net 3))
 (segment (start 143 39) (end 142.5 39.5) (width 0.45) (layer F.Cu) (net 3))
 (segment (start 141.5 42.5) (end 140.5 43.5) (width 0.45) (layer F.Cu) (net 3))
 (segment (start 138.5 47.5) (end 138.5 48.5) (width 0.45) (layer F.Cu) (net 3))
 (segment (start 146.5 38.38) (end 145.12 38.38) (width 0.45) (layer F.Cu) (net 3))
 (segment (start 144.5 39) (end 143 39) (width 0.45) (layer F.Cu) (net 3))
 (segment (start 145.12 38.38) (end 144.5 39) (width 0.45) (layer F.Cu) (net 3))
 (segment (start 139.5 46.5) (end 138.5 47.5) (width 0.45) (layer F.Cu) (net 3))
 (segment (start 139.5 45.5) (end 139.5 46.5) (width 0.45) (layer F.Cu) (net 3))
 (segment (start 138.5 48.5) (end 137.5 49.5) (width 0.45) (layer F.Cu) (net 3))
 (segment (start 137.5 49.5) (end 137.5 50.5) (width 0.45) (layer F.Cu) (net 3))
 (segment (start 137.5 50.5) (end 135 53) (width 0.45) (layer F.Cu) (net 3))
 (segment (start 131 52) (end 51.5 52) (width 0.45) (layer F.Cu) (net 2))
 (segment (start 134.5 52) (end 131 52) (width 0.45) (layer F.Cu) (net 2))
 (segment (start 136.5 50) (end 134.5 52) (width 0.45) (layer F.Cu) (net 2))
 (segment (start 137.5 48) (end 136.5 49) (width 0.45) (layer F.Cu) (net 2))
 (segment (start 145 36.5) (end 143 36.5) (width 0.45) (layer F.Cu) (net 2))
 (segment (start 137.5 47) (end 137.5 48) (width 0.45) (layer F.Cu) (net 2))
 (segment (start 143 36.5) (end 142.5 37) (width 0.45) (layer F.Cu) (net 2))
 (segment (start 146.5 35.84) (end 145.66 35.84) (width 0.45) (layer F.Cu) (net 2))
 (segment (start 141.5 40) (end 140.5 41) (width 0.45) (layer F.Cu) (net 2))
 (segment (start 145.66 35.84) (end 145 36.5) (width 0.45) (layer F.Cu) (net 2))
 (segment (start 141.5 39) (end 141.5 40) (width 0.45) (layer F.Cu) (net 2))
 (segment (start 140.5 41) (end 140.5 42) (width 0.45) (layer F.Cu) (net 2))
 (segment (start 136.5 49) (end 136.5 50) (width 0.45) (layer F.Cu) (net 2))
 (segment (start 142.5 38) (end 141.5 39) (width 0.45) (layer F.Cu) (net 2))
 (segment (start 140.5 42) (end 139.5 43) (width 0.45) (layer F.Cu) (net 2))
 (segment (start 139.5 43) (end 139.5 44) (width 0.45) (layer F.Cu) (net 2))
 (segment (start 142.5 37) (end 142.5 38) (width 0.45) (layer F.Cu) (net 2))
 (segment (start 139.5 44) (end 138.5 45) (width 0.45) (layer F.Cu) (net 2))
 (segment (start 138.5 46) (end 137.5 47) (width 0.45) (layer F.Cu) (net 2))
 (segment (start 138.5 45) (end 138.5 46) (width 0.45) (layer F.Cu) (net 2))
 (segment (start 135.5 49.5) (end 134 51) (width 0.45) (layer F.Cu) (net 1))
 (segment (start 135.5 48.5) (end 135.5 49.5) (width 0.45) (layer F.Cu) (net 1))
 (segment (start 137.5 44.5) (end 137.5 45.5) (width 0.45) (layer F.Cu) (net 1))
 (segment (start 143 34) (end 142.5 34.5) (width 0.45) (layer F.Cu) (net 1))
 (segment (start 51.5 51) (end 131 51) (width 0.45) (layer F.Cu) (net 1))
 (segment (start 146.5 33.3) (end 145.7 33.3) (width 0.45) (layer F.Cu) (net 1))
 (segment (start 145 34) (end 143 34) (width 0.45) (layer F.Cu) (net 1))
 (segment (start 145.7 33.3) (end 145 34) (width 0.45) (layer F.Cu) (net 1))
 (segment (start 138.5 42.5) (end 138.5 43.5) (width 0.45) (layer F.Cu) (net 1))
 (segment (start 138.5 43.5) (end 137.5 44.5) (width 0.45) (layer F.Cu) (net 1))
 (segment (start 131 51) (end 131.5 51) (width 0.45) (layer F.Cu) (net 1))
 (segment (start 142.5 34.5) (end 142.5 35.5) (width 0.45) (layer F.Cu) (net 1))
 (segment (start 141.5 37.5) (end 140.5 38.5) (width 0.45) (layer F.Cu) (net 1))
 (segment (start 136.5 46.5) (end 136.5 47.5) (width 0.45) (layer F.Cu) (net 1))
 (segment (start 137.5 45.5) (end 136.5 46.5) (width 0.45) (layer F.Cu) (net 1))
 (segment (start 142.5 35.5) (end 141.5 36.5) (width 0.45) (layer F.Cu) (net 1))
 (segment (start 141.5 36.5) (end 141.5 37.5) (width 0.45) (layer F.Cu) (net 1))
 (segment (start 139.5 41.5) (end 138.5 42.5) (width 0.45) (layer F.Cu) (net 1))
 (segment (start 136.5 47.5) (end 135.5 48.5) (width 0.45) (layer F.Cu) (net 1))
 (segment (start 140.5 38.5) (end 140.5 39.5) (width 0.45) (layer F.Cu) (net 1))
 (segment (start 134 51) (end 131 51) (width 0.45) (layer F.Cu) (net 1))
 (segment (start 140.5 39.5) (end 139.5 40.5) (width 0.45) (layer F.Cu) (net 1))
 (segment (start 139.5 40.5) (end 139.5 41.5) (width 0.45) (layer F.Cu) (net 1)))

